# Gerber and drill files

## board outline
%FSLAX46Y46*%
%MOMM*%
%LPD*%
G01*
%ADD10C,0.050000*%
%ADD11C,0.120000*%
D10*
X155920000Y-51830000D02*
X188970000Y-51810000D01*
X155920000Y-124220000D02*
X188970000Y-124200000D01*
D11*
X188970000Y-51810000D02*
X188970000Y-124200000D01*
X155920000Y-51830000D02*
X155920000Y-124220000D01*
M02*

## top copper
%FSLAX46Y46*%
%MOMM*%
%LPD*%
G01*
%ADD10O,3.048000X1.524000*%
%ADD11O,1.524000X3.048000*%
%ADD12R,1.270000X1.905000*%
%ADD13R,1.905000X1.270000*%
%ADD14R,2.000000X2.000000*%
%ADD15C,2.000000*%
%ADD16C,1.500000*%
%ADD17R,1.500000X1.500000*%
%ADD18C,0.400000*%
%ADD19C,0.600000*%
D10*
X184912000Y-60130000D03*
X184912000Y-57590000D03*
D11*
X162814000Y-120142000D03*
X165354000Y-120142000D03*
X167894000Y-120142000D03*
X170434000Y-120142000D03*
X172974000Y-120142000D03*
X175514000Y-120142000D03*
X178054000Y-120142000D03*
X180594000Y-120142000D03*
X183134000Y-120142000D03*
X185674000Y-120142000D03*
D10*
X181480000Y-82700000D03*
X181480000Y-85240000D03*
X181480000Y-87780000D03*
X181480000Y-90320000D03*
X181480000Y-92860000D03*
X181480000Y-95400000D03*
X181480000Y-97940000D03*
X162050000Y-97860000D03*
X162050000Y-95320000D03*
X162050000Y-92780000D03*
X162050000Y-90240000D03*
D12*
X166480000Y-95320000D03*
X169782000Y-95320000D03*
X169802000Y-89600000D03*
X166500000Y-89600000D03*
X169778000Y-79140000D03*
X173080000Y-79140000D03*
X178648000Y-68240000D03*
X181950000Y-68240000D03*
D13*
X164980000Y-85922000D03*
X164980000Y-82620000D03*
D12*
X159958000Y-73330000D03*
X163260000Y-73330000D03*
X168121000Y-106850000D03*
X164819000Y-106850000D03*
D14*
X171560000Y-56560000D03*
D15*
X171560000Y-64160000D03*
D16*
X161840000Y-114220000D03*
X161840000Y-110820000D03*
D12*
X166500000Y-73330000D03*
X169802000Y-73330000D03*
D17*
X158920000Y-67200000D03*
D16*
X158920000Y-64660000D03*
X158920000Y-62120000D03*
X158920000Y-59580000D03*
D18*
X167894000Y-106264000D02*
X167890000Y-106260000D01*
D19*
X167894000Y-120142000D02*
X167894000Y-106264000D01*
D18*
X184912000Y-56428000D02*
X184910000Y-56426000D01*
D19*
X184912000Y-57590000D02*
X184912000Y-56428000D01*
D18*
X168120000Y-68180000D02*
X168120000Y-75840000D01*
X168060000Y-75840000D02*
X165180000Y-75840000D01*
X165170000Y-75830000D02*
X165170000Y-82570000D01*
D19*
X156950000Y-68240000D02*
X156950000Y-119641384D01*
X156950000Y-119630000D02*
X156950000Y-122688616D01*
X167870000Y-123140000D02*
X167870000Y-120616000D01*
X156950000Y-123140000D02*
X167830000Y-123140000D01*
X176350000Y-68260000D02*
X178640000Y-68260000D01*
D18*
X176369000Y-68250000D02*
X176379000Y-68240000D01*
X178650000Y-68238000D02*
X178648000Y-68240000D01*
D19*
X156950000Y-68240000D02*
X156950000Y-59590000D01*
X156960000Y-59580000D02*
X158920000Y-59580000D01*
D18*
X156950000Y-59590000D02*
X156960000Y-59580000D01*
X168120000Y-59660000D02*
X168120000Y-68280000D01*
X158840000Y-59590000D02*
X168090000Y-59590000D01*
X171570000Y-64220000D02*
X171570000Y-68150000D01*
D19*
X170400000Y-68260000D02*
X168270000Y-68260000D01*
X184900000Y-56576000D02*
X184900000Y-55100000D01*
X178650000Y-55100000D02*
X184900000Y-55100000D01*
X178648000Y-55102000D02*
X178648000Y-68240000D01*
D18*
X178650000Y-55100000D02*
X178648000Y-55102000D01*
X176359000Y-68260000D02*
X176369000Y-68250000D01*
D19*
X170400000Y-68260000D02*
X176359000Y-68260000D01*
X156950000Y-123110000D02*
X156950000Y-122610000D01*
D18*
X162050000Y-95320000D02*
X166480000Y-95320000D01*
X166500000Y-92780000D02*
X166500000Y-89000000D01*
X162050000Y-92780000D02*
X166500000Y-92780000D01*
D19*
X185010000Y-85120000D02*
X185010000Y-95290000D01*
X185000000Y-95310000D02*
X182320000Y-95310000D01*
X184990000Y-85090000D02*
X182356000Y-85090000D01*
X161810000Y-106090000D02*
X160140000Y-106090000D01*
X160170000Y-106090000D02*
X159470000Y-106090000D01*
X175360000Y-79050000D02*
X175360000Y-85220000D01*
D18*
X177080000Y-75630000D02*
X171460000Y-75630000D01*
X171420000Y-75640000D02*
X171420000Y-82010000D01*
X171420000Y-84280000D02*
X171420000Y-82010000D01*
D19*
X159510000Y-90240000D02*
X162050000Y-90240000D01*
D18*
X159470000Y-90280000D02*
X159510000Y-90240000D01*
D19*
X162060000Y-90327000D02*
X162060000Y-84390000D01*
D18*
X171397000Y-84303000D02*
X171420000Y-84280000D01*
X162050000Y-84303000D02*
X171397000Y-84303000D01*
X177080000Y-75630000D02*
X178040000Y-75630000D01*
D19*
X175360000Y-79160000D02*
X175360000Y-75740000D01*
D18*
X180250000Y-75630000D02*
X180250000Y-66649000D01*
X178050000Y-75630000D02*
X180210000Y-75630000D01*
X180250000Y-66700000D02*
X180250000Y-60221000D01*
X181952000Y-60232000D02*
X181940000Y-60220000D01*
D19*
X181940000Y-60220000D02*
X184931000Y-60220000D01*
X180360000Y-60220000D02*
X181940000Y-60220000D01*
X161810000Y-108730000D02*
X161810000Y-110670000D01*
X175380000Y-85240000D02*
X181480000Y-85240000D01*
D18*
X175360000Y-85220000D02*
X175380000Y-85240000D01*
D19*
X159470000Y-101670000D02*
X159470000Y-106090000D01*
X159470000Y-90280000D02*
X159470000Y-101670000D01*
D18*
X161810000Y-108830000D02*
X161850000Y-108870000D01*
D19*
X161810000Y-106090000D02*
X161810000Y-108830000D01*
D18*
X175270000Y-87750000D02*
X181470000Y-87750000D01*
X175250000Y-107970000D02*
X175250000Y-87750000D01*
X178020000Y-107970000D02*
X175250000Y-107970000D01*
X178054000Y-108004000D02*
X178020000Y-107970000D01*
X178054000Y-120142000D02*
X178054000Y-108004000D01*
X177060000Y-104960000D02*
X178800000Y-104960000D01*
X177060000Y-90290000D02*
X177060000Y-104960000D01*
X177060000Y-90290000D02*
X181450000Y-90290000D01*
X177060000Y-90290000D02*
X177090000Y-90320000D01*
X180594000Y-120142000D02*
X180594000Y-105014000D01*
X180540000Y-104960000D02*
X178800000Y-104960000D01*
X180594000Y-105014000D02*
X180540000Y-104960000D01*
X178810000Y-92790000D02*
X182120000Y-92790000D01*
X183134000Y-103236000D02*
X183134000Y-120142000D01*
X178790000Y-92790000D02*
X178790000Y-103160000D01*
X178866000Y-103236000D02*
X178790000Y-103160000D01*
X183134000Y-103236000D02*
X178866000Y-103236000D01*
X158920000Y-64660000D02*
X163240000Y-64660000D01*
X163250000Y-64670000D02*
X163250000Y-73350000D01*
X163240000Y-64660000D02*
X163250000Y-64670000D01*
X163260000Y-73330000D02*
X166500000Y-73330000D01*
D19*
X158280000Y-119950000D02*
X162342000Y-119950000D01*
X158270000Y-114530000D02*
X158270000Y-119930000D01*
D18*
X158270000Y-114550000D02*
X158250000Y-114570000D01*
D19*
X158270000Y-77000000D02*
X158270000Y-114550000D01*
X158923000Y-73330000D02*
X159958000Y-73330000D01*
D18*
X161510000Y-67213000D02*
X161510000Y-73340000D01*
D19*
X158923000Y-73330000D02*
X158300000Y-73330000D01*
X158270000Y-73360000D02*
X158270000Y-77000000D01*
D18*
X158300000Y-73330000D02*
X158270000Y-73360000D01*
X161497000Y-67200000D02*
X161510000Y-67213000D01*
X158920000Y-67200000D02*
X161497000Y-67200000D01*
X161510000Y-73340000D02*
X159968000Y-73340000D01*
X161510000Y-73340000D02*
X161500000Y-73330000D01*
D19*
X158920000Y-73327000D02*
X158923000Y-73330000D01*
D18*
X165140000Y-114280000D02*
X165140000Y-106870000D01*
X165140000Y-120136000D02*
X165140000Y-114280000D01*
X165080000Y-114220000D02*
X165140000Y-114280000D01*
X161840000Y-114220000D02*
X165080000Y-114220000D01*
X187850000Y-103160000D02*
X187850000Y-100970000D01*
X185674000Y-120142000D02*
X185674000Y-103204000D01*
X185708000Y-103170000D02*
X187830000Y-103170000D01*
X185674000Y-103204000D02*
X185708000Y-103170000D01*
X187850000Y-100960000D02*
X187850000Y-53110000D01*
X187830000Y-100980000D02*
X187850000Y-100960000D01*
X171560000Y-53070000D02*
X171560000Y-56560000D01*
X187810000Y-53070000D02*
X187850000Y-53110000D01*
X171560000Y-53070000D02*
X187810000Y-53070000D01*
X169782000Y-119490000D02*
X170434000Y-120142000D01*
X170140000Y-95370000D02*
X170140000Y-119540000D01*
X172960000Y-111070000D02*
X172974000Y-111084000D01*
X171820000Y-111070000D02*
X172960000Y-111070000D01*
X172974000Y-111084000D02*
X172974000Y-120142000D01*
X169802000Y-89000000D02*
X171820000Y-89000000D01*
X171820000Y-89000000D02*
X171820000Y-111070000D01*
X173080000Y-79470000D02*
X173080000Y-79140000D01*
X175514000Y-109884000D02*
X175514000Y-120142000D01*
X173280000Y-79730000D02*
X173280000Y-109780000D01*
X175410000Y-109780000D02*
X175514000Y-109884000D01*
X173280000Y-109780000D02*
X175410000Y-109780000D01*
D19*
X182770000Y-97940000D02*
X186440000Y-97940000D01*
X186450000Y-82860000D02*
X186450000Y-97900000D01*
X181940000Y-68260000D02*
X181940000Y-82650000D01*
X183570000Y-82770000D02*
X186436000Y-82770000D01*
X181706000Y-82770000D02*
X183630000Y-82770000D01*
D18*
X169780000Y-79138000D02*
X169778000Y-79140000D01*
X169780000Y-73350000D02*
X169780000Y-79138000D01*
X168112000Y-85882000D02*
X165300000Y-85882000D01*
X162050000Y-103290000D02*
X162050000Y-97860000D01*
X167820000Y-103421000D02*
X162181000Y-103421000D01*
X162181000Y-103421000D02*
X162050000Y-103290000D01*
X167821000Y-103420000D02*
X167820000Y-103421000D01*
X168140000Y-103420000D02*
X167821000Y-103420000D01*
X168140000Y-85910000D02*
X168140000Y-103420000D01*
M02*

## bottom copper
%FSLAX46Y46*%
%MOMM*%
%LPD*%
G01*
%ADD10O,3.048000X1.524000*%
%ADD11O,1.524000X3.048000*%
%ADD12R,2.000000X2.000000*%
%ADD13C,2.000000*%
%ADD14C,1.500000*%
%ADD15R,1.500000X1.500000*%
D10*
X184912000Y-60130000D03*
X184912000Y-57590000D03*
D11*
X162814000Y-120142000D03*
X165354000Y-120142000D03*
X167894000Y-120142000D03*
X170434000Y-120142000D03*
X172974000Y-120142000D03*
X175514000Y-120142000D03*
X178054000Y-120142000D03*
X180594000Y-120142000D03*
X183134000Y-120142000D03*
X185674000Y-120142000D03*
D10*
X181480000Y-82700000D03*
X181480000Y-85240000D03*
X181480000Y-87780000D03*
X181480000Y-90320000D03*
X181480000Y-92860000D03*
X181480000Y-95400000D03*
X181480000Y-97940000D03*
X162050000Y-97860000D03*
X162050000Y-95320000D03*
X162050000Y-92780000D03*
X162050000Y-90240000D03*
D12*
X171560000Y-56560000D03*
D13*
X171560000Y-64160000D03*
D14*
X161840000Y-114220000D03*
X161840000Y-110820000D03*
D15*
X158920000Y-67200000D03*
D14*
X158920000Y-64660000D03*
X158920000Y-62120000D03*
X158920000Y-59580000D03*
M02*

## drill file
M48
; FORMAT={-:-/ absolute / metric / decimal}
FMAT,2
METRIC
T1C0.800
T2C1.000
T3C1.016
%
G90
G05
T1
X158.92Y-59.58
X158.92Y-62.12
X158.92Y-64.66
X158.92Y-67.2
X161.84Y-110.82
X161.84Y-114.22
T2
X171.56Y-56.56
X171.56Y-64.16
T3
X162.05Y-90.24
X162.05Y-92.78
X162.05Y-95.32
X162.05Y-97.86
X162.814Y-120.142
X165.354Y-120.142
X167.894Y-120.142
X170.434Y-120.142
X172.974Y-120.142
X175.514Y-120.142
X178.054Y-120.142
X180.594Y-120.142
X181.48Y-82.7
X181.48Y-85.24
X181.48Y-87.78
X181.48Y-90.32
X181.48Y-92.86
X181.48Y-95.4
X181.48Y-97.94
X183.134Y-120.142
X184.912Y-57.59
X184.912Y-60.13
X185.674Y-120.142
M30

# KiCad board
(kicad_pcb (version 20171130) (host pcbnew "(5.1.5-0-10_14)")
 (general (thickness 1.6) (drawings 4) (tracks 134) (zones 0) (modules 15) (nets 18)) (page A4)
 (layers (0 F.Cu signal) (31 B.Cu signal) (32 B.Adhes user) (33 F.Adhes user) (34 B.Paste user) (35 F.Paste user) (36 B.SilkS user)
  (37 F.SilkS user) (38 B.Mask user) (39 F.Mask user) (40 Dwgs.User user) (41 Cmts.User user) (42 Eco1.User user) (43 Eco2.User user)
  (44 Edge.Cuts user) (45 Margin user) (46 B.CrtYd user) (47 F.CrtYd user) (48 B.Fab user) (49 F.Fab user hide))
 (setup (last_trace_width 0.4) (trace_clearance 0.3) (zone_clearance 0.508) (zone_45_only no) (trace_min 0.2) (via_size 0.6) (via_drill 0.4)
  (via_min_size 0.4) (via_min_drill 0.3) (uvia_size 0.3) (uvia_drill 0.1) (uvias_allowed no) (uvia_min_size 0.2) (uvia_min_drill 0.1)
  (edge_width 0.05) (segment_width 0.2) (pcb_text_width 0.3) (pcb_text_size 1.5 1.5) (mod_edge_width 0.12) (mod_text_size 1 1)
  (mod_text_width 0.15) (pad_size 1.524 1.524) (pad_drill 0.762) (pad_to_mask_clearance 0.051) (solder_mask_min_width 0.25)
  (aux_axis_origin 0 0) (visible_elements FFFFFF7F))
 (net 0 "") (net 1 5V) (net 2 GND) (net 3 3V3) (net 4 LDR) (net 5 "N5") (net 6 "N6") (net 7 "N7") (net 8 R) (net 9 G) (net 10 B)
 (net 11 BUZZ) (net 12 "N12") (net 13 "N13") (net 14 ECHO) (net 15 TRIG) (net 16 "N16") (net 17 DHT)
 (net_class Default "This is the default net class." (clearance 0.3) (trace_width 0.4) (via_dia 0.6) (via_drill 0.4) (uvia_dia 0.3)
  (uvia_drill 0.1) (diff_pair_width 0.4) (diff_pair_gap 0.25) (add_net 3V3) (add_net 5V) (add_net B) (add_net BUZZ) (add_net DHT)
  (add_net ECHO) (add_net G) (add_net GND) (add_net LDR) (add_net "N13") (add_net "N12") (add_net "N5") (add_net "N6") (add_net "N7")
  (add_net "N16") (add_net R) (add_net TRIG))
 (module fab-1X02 (layer F.Cu) (at 184.912 58.86 90)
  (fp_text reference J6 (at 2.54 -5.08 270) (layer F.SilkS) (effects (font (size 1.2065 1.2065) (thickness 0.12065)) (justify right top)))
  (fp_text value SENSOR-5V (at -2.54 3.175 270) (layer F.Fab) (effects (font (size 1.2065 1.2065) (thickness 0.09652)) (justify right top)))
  (pad 1 thru_hole oval (at -1.27 0 180) (size 3.048 1.524) (drill 1.016) (layers *.Cu *.Mask) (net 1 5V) (solder_mask_margin 0.1016))
  (pad 2 thru_hole oval (at 1.27 0 180) (size 3.048 1.524) (drill 1.016) (layers *.Cu *.Mask) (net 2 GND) (solder_mask_margin 0.1016)))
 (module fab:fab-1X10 (layer F.Cu) (at 174.244 120.142)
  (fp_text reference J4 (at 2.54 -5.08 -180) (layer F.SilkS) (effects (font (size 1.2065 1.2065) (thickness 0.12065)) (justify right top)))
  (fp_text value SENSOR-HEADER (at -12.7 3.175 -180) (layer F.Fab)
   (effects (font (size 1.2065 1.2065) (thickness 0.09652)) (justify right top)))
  (pad 1 thru_hole oval (at -11.43 0 90) (size 3.048 1.524) (drill 1.016) (layers *.Cu *.Mask) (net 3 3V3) (solder_mask_margin 0.1016))
  (pad 2 thru_hole oval (at -8.89 0 90) (size 3.048 1.524) (drill 1.016) (layers *.Cu *.Mask) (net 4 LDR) (solder_mask_margin 0.1016))
  (pad 3 thru_hole oval (at -6.35 0 90) (size 3.048 1.524) (drill 1.016) (layers *.Cu *.Mask) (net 2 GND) (solder_mask_margin 0.1016))
  (pad 4 thru_hole oval (at -3.81 0 90) (size 3.048 1.524) (drill 1.016) (layers *.Cu *.Mask) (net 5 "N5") (solder_mask_margin 0.1016))
  (pad 5 thru_hole oval (at -1.27 0 90) (size 3.048 1.524) (drill 1.016) (layers *.Cu *.Mask) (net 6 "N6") (solder_mask_margin 0.1016))
  (pad 6 thru_hole oval (at 1.27 0 90) (size 3.048 1.524) (drill 1.016) (layers *.Cu *.Mask) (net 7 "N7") (solder_mask_margin 0.1016))
  (pad 7 thru_hole oval (at 3.81 0 90) (size 3.048 1.524) (drill 1.016) (layers *.Cu *.Mask) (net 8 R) (solder_mask_margin 0.1016))
  (pad 8 thru_hole oval (at 6.35 0 90) (size 3.048 1.524) (drill 1.016) (layers *.Cu *.Mask) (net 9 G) (solder_mask_margin 0.1016))
  (pad 9 thru_hole oval (at 8.89 0 90) (size 3.048 1.524) (drill 1.016) (layers *.Cu *.Mask) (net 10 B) (solder_mask_margin 0.1016))
  (pad 10 thru_hole oval (at 11.43 0 90) (size 3.048 1.524) (drill 1.016) (layers *.Cu *.Mask) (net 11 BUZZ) (solder_mask_margin 0.1016)))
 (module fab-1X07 (layer F.Cu) (at 181.48 90.32 270)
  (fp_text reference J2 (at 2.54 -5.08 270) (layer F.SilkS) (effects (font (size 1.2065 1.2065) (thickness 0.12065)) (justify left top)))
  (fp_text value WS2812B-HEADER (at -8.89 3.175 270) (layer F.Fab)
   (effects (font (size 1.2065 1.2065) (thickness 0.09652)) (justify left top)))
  (pad 1 thru_hole oval (at -7.62 0) (size 3.048 1.524) (drill 1.016) (layers *.Cu *.Mask) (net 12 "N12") (solder_mask_margin 0.1016))
  (pad 2 thru_hole oval (at -5.08 0) (size 3.048 1.524) (drill 1.016) (layers *.Cu *.Mask) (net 1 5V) (solder_mask_margin 0.1016))
  (pad 3 thru_hole oval (at -2.54 0) (size 3.048 1.524) (drill 1.016) (layers *.Cu *.Mask) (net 8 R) (solder_mask_margin 0.1016))
  (pad 4 thru_hole oval (at 0 0) (size 3.048 1.524) (drill 1.016) (layers *.Cu *.Mask) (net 9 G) (solder_mask_margin 0.1016))
  (pad 5 thru_hole oval (at 2.54 0) (size 3.048 1.524) (drill 1.016) (layers *.Cu *.Mask) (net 10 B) (solder_mask_margin 0.1016))
  (pad 6 thru_hole oval (at 5.08 0) (size 3.048 1.524) (drill 1.016) (layers *.Cu *.Mask) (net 1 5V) (solder_mask_margin 0.1016))
  (pad 7 thru_hole oval (at 7.62 0) (size 3.048 1.524) (drill 1.016) (layers *.Cu *.Mask) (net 12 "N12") (solder_mask_margin 0.1016)))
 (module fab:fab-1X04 (layer F.Cu) (at 162.05 94.05 90)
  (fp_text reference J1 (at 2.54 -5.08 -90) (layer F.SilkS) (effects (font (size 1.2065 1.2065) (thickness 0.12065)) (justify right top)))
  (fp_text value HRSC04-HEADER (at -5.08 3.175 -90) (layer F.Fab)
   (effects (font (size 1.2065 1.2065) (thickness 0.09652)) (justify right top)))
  (pad 1 thru_hole oval (at -3.81 0 180) (size 3.048 1.524) (drill 1.016) (layers *.Cu *.Mask) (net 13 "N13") (solder_mask_margin 0.1016))
  (pad 2 thru_hole oval (at -1.27 0 180) (size 3.048 1.524) (drill 1.016) (layers *.Cu *.Mask) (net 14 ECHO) (solder_mask_margin 0.1016))
  (pad 3 thru_hole oval (at 1.27 0 180) (size 3.048 1.524) (drill 1.016) (layers *.Cu *.Mask) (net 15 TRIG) (solder_mask_margin 0.1016))
  (pad 4 thru_hole oval (at 3.81 0 180) (size 3.048 1.524) (drill 1.016) (layers *.Cu *.Mask) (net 1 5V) (solder_mask_margin 0.1016)))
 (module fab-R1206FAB (layer F.Cu) (at 168.131 95.32)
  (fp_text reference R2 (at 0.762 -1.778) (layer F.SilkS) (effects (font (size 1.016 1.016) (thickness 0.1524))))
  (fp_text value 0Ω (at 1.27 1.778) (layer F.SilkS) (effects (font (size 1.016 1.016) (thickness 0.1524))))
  (pad 1 smd rect (at -1.651 0) (size 1.27 1.905) (layers F.Cu F.Paste F.Mask) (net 14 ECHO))
  (pad 2 smd rect (at 1.651 0) (size 1.27 1.905) (layers F.Cu F.Paste F.Mask) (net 5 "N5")))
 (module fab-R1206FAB (layer F.Cu) (at 168.151 89.6)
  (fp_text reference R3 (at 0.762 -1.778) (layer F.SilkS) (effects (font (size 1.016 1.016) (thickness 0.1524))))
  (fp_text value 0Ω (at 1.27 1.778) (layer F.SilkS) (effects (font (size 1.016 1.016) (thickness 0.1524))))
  (pad 2 smd rect (at 1.651 0) (size 1.27 1.905) (layers F.Cu F.Paste F.Mask) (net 6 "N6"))
  (pad 1 smd rect (at -1.651 0) (size 1.27 1.905) (layers F.Cu F.Paste F.Mask) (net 15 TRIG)))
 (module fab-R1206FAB (layer F.Cu) (at 171.429 79.14)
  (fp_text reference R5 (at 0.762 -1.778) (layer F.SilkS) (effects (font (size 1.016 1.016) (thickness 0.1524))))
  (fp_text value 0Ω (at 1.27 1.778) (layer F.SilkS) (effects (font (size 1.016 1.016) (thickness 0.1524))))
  (pad 1 smd rect (at -1.651 0) (size 1.27 1.905) (layers F.Cu F.Paste F.Mask) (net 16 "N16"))
  (pad 2 smd rect (at 1.651 0) (size 1.27 1.905) (layers F.Cu F.Paste F.Mask) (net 7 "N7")))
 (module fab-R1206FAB (layer F.Cu) (at 180.299 68.24)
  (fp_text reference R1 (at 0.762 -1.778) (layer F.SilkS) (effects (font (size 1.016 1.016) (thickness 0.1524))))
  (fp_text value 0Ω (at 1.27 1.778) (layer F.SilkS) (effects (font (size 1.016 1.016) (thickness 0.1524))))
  (pad 1 smd rect (at -1.651 0) (size 1.27 1.905) (layers F.Cu F.Paste F.Mask) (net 2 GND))
  (pad 2 smd rect (at 1.651 0) (size 1.27 1.905) (layers F.Cu F.Paste F.Mask) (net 12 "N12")))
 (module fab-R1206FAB (layer F.Cu) (at 164.98 84.271 90)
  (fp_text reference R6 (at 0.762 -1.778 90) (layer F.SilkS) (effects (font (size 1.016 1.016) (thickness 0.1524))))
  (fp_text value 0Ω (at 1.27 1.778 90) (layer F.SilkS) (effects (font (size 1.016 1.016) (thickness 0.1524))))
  (pad 1 smd rect (at -1.651 0 90) (size 1.27 1.905) (layers F.Cu F.Paste F.Mask) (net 13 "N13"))
  (pad 2 smd rect (at 1.651 0 90) (size 1.27 1.905) (layers F.Cu F.Paste F.Mask) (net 2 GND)))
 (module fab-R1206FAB (layer F.Cu) (at 161.609 73.33)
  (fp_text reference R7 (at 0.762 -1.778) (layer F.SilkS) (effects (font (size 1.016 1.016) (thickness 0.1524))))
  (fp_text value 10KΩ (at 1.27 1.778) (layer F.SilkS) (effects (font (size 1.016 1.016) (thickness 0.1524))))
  (pad 1 smd rect (at -1.651 0) (size 1.27 1.905) (layers F.Cu F.Paste F.Mask) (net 3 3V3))
  (pad 2 smd rect (at 1.651 0) (size 1.27 1.905) (layers F.Cu F.Paste F.Mask) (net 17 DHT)))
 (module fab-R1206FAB (layer F.Cu) (at 166.47 106.85)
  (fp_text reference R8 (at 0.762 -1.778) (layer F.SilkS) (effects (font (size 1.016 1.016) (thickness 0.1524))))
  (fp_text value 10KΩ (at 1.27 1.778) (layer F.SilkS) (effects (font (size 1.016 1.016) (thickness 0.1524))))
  (pad 2 smd rect (at 1.651 0) (size 1.27 1.905) (layers F.Cu F.Paste F.Mask) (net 2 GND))
  (pad 1 smd rect (at -1.651 0) (size 1.27 1.905) (layers F.Cu F.Paste F.Mask) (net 4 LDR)))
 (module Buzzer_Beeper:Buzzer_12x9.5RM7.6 (layer F.Cu) (at 171.56 56.56 270)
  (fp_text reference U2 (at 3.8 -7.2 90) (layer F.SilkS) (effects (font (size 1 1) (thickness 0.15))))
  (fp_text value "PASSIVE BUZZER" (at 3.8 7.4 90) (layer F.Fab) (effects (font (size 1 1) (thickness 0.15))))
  (pad 1 thru_hole rect (at 0 0 270) (size 2 2) (drill 1) (layers *.Cu *.Mask) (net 11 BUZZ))
  (pad 2 thru_hole circle (at 7.6 0 270) (size 2 2) (drill 1) (layers *.Cu *.Mask) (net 2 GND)))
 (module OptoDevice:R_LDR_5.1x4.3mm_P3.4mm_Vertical (layer F.Cu) (at 161.84 114.22 90)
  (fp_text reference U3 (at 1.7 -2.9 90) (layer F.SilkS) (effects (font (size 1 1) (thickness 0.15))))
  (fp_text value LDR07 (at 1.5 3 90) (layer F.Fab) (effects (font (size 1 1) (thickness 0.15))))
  (pad 1 thru_hole circle (at 0 0 90) (size 1.5 1.5) (drill 0.8) (layers *.Cu *.Mask) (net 4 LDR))
  (pad 2 thru_hole circle (at 3.4 0 90) (size 1.5 1.5) (drill 0.8) (layers *.Cu *.Mask) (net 1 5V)))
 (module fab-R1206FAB (layer F.Cu) (at 168.151 73.33)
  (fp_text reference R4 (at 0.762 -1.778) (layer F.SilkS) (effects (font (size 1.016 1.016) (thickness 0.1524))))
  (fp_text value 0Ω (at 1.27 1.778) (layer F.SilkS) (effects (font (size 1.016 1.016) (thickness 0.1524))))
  (pad 1 smd rect (at -1.651 0) (size 1.27 1.905) (layers F.Cu F.Paste F.Mask) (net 17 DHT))
  (pad 2 smd rect (at 1.651 0) (size 1.27 1.905) (layers F.Cu F.Paste F.Mask) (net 16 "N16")))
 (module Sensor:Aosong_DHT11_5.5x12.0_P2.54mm (layer F.Cu) (at 158.92 67.2 180)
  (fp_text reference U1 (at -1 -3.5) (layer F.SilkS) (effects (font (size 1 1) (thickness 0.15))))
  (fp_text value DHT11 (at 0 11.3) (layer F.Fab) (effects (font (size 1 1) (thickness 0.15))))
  (pad 1 thru_hole rect (at 0 0 180) (size 1.5 1.5) (drill 0.8) (layers *.Cu *.Mask) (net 3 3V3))
  (pad 2 thru_hole circle (at 0 2.54 180) (size 1.5 1.5) (drill 0.8) (layers *.Cu *.Mask) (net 17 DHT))
  (pad 3 thru_hole circle (at 0 5.08 180) (size 1.5 1.5) (drill 0.8) (layers *.Cu *.Mask))
  (pad 4 thru_hole circle (at 0 7.62 180) (size 1.5 1.5) (drill 0.8) (layers *.Cu *.Mask) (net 2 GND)))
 (gr_line (start 155.92 51.83) (end 188.97 51.81) (layer Edge.Cuts) (width 0.05))
 (gr_line (start 155.92 124.22) (end 188.97 124.2) (layer Edge.Cuts) (width 0.05))
 (gr_line (start 188.97 51.81) (end 188.97 124.2) (layer Edge.Cuts) (width 0.12))
 (gr_line (start 155.92 51.83) (end 155.92 124.22) (layer Edge.Cuts) (width 0.12))
 (segment (start 167.894 106.264) (end 167.89 106.26) (width 0.4) (layer F.Cu) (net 2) (status 30))
 (segment (start 167.894 120.142) (end 167.894 106.264) (width 0.6) (layer F.Cu) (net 2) (status 30))
 (segment (start 184.912 56.428) (end 184.91 56.426) (width 0.4) (layer F.Cu) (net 2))
 (segment (start 184.912 57.59) (end 184.912 56.428) (width 0.6) (layer F.Cu) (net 2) (status 10))
 (segment (start 168.12 68.18) (end 168.12 75.84) (width 0.4) (layer F.Cu) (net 2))
 (segment (start 168.06 75.84) (end 165.18 75.84) (width 0.4) (layer F.Cu) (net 2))
 (segment (start 165.17 75.83) (end 165.17 82.57) (width 0.4) (layer F.Cu) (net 2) (status 20))
 (segment (start 156.95 68.24) (end 156.95 119.641384) (width 0.6) (layer F.Cu) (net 2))
 (segment (start 156.95 119.63) (end 156.95 122.688616) (width 0.6) (layer F.Cu) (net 2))
 (segment (start 167.87 123.14) (end 167.87 120.616) (width 0.6) (layer F.Cu) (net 2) (status 20))
 (segment (start 156.95 123.14) (end 167.83 123.14) (width 0.6) (layer F.Cu) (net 2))
 (segment (start 176.35 68.26) (end 178.64 68.26) (width 0.6) (layer F.Cu) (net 2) (status 20))
 (segment (start 176.369 68.25) (end 176.379 68.24) (width 0.4) (layer F.Cu) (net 2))
 (segment (start 178.65 68.238) (end 178.648 68.24) (width 0.4) (layer F.Cu) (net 2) (status 30))
 (segment (start 156.95 68.24) (end 156.95 59.59) (width 0.6) (layer F.Cu) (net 2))
 (segment (start 156.96 59.58) (end 158.92 59.58) (width 0.6) (layer F.Cu) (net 2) (status 20))
 (segment (start 156.95 59.59) (end 156.96 59.58) (width 0.4) (layer F.Cu) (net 2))
 (segment (start 168.12 59.66) (end 168.12 68.28) (width 0.4) (layer F.Cu) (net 2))
 (segment (start 158.84 59.59) (end 168.09 59.59) (width 0.4) (layer F.Cu) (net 2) (status 10))
 (segment (start 171.57 64.22) (end 171.57 68.15) (width 0.4) (layer F.Cu) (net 2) (status 10))
 (segment (start 170.4 68.26) (end 168.27 68.26) (width 0.6) (layer F.Cu) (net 2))
 (segment (start 184.9 56.576) (end 184.9 55.1) (width 0.6) (layer F.Cu) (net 2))
 (segment (start 178.65 55.1) (end 184.9 55.1) (width 0.6) (layer F.Cu) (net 2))
 (segment (start 178.648 55.102) (end 178.648 68.24) (width 0.6) (layer F.Cu) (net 2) (status 20))
 (segment (start 178.65 55.1) (end 178.648 55.102) (width 0.4) (layer F.Cu) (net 2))
 (segment (start 176.359 68.26) (end 176.369 68.25) (width 0.4) (layer F.Cu) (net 2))
 (segment (start 170.4 68.26) (end 176.359 68.26) (width 0.6) (layer F.Cu) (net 2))
 (segment (start 156.95 123.11) (end 156.95 122.61) (width 0.6) (layer F.Cu) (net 2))
 (segment (start 162.05 95.32) (end 166.48 95.32) (width 0.4) (layer F.Cu) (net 14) (status 30))
 (segment (start 166.5 92.78) (end 166.5 89) (width 0.4) (layer F.Cu) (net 15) (status 20))
 (segment (start 162.05 92.78) (end 166.5 92.78) (width 0.4) (layer F.Cu) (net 15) (status 10))
 (segment (start 185.01 85.12) (end 185.01 95.29) (width 0.6) (layer F.Cu) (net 1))
 (segment (start 185 95.31) (end 182.32 95.31) (width 0.6) (layer F.Cu) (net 1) (status 20))
 (segment (start 184.99 85.09) (end 182.356 85.09) (width 0.6) (layer F.Cu) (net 1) (status 20))
 (segment (start 161.81 106.09) (end 160.14 106.09) (width 0.6) (layer F.Cu) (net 1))
 (segment (start 160.17 106.09) (end 159.47 106.09) (width 0.6) (layer F.Cu) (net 1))
 (segment (start 175.36 79.05) (end 175.36 85.22) (width 0.6) (layer F.Cu) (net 1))
 (segment (start 177.08 75.63) (end 171.46 75.63) (width 0.4) (layer F.Cu) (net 1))
 (segment (start 171.42 75.64) (end 171.42 82.01) (width 0.4) (layer F.Cu) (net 1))
 (segment (start 171.42 84.28) (end 171.42 82.01) (width 0.4) (layer F.Cu) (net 1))
 (segment (start 159.51 90.24) (end 162.05 90.24) (width 0.6) (layer F.Cu) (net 1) (status 20))
 (segment (start 159.47 90.28) (end 159.51 90.24) (width 0.4) (layer F.Cu) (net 1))
 (segment (start 162.06 90.327) (end 162.06 84.39) (width 0.6) (layer F.Cu) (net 1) (status 10))
 (segment (start 171.397 84.303) (end 171.42 84.28) (width 0.4) (layer F.Cu) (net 1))
 (segment (start 162.05 84.303) (end 171.397 84.303) (width 0.4) (layer F.Cu) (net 1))
 (segment (start 177.08 75.63) (end 178.04 75.63) (width 0.4) (layer F.Cu) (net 1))
 (segment (start 175.36 79.16) (end 175.36 75.74) (width 0.6) (layer F.Cu) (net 1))
 (segment (start 180.25 75.63) (end 180.25 66.649) (width 0.4) (layer F.Cu) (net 1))
 (segment (start 178.05 75.63) (end 180.21 75.63) (width 0.4) (layer F.Cu) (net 1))
 (segment (start 180.25 66.7) (end 180.25 60.221) (width 0.4) (layer F.Cu) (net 1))
 (segment (start 181.952 60.232) (end 181.94 60.22) (width 0.4) (layer F.Cu) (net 1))
 (segment (start 181.94 60.22) (end 184.931 60.22) (width 0.6) (layer F.Cu) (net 1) (status 20))
 (segment (start 180.36 60.22) (end 181.94 60.22) (width 0.6) (layer F.Cu) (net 1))
 (segment (start 161.81 108.73) (end 161.81 110.67) (width 0.6) (layer F.Cu) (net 1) (status 20))
 (segment (start 175.38 85.24) (end 181.48 85.24) (width 0.6) (layer F.Cu) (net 1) (status 20))
 (segment (start 175.36 85.22) (end 175.38 85.24) (width 0.4) (layer F.Cu) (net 1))
 (segment (start 159.47 101.67) (end 159.47 106.09) (width 0.6) (layer F.Cu) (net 1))
 (segment (start 159.47 90.28) (end 159.47 101.67) (width 0.6) (layer F.Cu) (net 1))
 (segment (start 161.81 108.83) (end 161.85 108.87) (width 0.4) (layer F.Cu) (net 1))
 (segment (start 161.81 106.09) (end 161.81 108.83) (width 0.6) (layer F.Cu) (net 1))
 (segment (start 175.27 87.75) (end 181.47 87.75) (width 0.4) (layer F.Cu) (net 8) (status 20))
 (segment (start 175.25 107.97) (end 175.25 87.75) (width 0.4) (layer F.Cu) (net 8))
 (segment (start 178.02 107.97) (end 175.25 107.97) (width 0.4) (layer F.Cu) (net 8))
 (segment (start 178.054 108.004) (end 178.02 107.97) (width 0.4) (layer F.Cu) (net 8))
 (segment (start 178.054 120.142) (end 178.054 108.004) (width 0.4) (layer F.Cu) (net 8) (status 10))
 (segment (start 177.06 104.96) (end 178.8 104.96) (width 0.4) (layer F.Cu) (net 9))
 (segment (start 177.06 90.29) (end 177.06 104.96) (width 0.4) (layer F.Cu) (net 9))
 (segment (start 177.06 90.29) (end 181.45 90.29) (width 0.4) (layer F.Cu) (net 9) (status 20))
 (segment (start 177.06 90.29) (end 177.09 90.32) (width 0.4) (layer F.Cu) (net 9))
 (segment (start 180.594 120.142) (end 180.594 105.014) (width 0.4) (layer F.Cu) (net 9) (status 10))
 (segment (start 180.54 104.96) (end 178.8 104.96) (width 0.4) (layer F.Cu) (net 9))
 (segment (start 180.594 105.014) (end 180.54 104.96) (width 0.4) (layer F.Cu) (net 9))
 (segment (start 178.81 92.79) (end 182.12 92.79) (width 0.4) (layer F.Cu) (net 10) (status 20))
 (segment (start 183.134 103.236) (end 183.134 120.142) (width 0.4) (layer F.Cu) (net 10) (status 20))
 (segment (start 178.79 92.79) (end 178.79 103.16) (width 0.4) (layer F.Cu) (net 10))
 (segment (start 178.866 103.236) (end 178.79 103.16) (width 0.4) (layer F.Cu) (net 10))
 (segment (start 183.134 103.236) (end 178.866 103.236) (width 0.4) (layer F.Cu) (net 10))
 (segment (start 158.92 64.66) (end 163.24 64.66) (width 0.4) (layer F.Cu) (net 17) (status 10))
 (segment (start 163.25 64.67) (end 163.25 73.35) (width 0.4) (layer F.Cu) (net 17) (status 20))
 (segment (start 163.24 64.66) (end 163.25 64.67) (width 0.4) (layer F.Cu) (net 17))
 (segment (start 163.26 73.33) (end 166.5 73.33) (width 0.4) (layer F.Cu) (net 17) (status 30))
 (segment (start 158.28 119.95) (end 162.342 119.95) (width 0.6) (layer F.Cu) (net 3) (status 20))
 (segment (start 158.27 114.53) (end 158.27 119.93) (width 0.6) (layer F.Cu) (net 3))
 (segment (start 158.27 114.55) (end 158.25 114.57) (width 0.4) (layer F.Cu) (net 3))
 (segment (start 158.27 77) (end 158.27 114.55) (width 0.6) (layer F.Cu) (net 3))
 (segment (start 158.923 73.33) (end 159.958 73.33) (width 0.6) (layer F.Cu) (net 3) (status 20))
 (segment (start 161.51 67.213) (end 161.51 73.34) (width 0.4) (layer F.Cu) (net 3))
 (segment (start 158.923 73.33) (end 158.3 73.33) (width 0.6) (layer F.Cu) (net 3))
 (segment (start 158.27 73.36) (end 158.27 77) (width 0.6) (layer F.Cu) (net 3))
 (segment (start 158.3 73.33) (end 158.27 73.36) (width 0.4) (layer F.Cu) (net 3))
 (segment (start 161.497 67.2) (end 161.51 67.213) (width 0.4) (layer F.Cu) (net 3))
 (segment (start 158.92 67.2) (end 161.497 67.2) (width 0.4) (layer F.Cu) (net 3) (status 10))
 (segment (start 161.51 73.34) (end 159.968 73.34) (width 0.4) (layer F.Cu) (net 3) (status 20))
 (segment (start 161.51 73.34) (end 161.5 73.33) (width 0.4) (layer F.Cu) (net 3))
 (segment (start 158.92 73.327) (end 158.923 73.33) (width 0.6) (layer F.Cu) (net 3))
 (segment (start 165.14 114.28) (end 165.14 106.87) (width 0.4) (layer F.Cu) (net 4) (status 20))
 (segment (start 165.14 120.136) (end 165.14 114.28) (width 0.4) (layer F.Cu) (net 4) (status 10))
 (segment (start 165.08 114.22) (end 165.14 114.28) (width 0.4) (layer F.Cu) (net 4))
 (segment (start 161.84 114.22) (end 165.08 114.22) (width 0.4) (layer F.Cu) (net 4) (status 10))
 (segment (start 187.85 103.16) (end 187.85 100.97) (width 0.4) (layer F.Cu) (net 11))
 (segment (start 185.674 120.142) (end 185.674 103.204) (width 0.4) (layer F.Cu) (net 11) (status 10))
 (segment (start 185.708 103.17) (end 187.83 103.17) (width 0.4) (layer F.Cu) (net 11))
 (segment (start 185.674 103.204) (end 185.708 103.17) (width 0.4) (layer F.Cu) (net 11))
 (segment (start 187.85 100.96) (end 187.85 53.11) (width 0.4) (layer F.Cu) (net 11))
 (segment (start 187.83 100.98) (end 187.85 100.96) (width 0.4) (layer F.Cu) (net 11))
 (segment (start 171.56 53.07) (end 171.56 56.56) (width 0.4) (layer F.Cu) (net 11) (status 20))
 (segment (start 187.81 53.07) (end 187.85 53.11) (width 0.4) (layer F.Cu) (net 11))
 (segment (start 171.56 53.07) (end 187.81 53.07) (width 0.4) (layer F.Cu) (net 11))
 (segment (start 169.782 119.49) (end 170.434 120.142) (width 0.4) (layer F.Cu) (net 5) (status 30))
 (segment (start 170.14 95.37) (end 170.14 119.54) (width 0.4) (layer F.Cu) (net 5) (status 30))
 (segment (start 172.96 111.07) (end 172.974 111.084) (width 0.4) (layer F.Cu) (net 6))
 (segment (start 171.82 111.07) (end 172.96 111.07) (width 0.4) (layer F.Cu) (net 6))
 (segment (start 172.974 111.084) (end 172.974 120.142) (width 0.4) (layer F.Cu) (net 6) (status 20))
 (segment (start 169.802 89) (end 171.82 89) (width 0.4) (layer F.Cu) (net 6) (status 10))
 (segment (start 171.82 89) (end 171.82 111.07) (width 0.4) (layer F.Cu) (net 6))
 (segment (start 173.08 79.47) (end 173.08 79.14) (width 0.4) (layer F.Cu) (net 7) (status 30))
 (segment (start 175.514 109.884) (end 175.514 120.142) (width 0.4) (layer F.Cu) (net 7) (status 20))
 (segment (start 173.28 79.73) (end 173.28 109.78) (width 0.4) (layer F.Cu) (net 7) (status 10))
 (segment (start 175.41 109.78) (end 175.514 109.884) (width 0.4) (layer F.Cu) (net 7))
 (segment (start 173.28 109.78) (end 175.41 109.78) (width 0.4) (layer F.Cu) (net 7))
 (segment (start 182.77 97.94) (end 186.44 97.94) (width 0.6) (layer F.Cu) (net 12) (status 10))
 (segment (start 186.45 82.86) (end 186.45 97.9) (width 0.6) (layer F.Cu) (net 12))
 (segment (start 181.94 68.26) (end 181.94 82.65) (width 0.6) (layer F.Cu) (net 12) (status 30))
 (segment (start 183.57 82.77) (end 186.436 82.77) (width 0.6) (layer F.Cu) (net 12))
 (segment (start 181.706 82.77) (end 183.63 82.77) (width 0.6) (layer F.Cu) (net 12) (status 10))
 (segment (start 169.78 79.138) (end 169.778 79.14) (width 0.4) (layer F.Cu) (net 16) (status 30))
 (segment (start 169.78 73.35) (end 169.78 79.138) (width 0.4) (layer F.Cu) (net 16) (status 30))
 (segment (start 168.112 85.882) (end 165.3 85.882) (width 0.4) (layer F.Cu) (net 13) (status 20))
 (segment (start 162.05 103.29) (end 162.05 97.86) (width 0.4) (layer F.Cu) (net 13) (status 20))
 (segment (start 167.82 103.421) (end 162.181 103.421) (width 0.4) (layer F.Cu) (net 13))
 (segment (start 162.181 103.421) (end 162.05 103.29) (width 0.4) (layer F.Cu) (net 13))
 (segment (start 167.821 103.42) (end 167.82 103.421) (width 0.4) (layer F.Cu) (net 13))
 (segment (start 168.14 103.42) (end 167.821 103.42) (width 0.4) (layer F.Cu) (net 13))
 (segment (start 168.14 85.91) (end 168.14 103.42) (width 0.4) (layer F.Cu) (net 13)))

